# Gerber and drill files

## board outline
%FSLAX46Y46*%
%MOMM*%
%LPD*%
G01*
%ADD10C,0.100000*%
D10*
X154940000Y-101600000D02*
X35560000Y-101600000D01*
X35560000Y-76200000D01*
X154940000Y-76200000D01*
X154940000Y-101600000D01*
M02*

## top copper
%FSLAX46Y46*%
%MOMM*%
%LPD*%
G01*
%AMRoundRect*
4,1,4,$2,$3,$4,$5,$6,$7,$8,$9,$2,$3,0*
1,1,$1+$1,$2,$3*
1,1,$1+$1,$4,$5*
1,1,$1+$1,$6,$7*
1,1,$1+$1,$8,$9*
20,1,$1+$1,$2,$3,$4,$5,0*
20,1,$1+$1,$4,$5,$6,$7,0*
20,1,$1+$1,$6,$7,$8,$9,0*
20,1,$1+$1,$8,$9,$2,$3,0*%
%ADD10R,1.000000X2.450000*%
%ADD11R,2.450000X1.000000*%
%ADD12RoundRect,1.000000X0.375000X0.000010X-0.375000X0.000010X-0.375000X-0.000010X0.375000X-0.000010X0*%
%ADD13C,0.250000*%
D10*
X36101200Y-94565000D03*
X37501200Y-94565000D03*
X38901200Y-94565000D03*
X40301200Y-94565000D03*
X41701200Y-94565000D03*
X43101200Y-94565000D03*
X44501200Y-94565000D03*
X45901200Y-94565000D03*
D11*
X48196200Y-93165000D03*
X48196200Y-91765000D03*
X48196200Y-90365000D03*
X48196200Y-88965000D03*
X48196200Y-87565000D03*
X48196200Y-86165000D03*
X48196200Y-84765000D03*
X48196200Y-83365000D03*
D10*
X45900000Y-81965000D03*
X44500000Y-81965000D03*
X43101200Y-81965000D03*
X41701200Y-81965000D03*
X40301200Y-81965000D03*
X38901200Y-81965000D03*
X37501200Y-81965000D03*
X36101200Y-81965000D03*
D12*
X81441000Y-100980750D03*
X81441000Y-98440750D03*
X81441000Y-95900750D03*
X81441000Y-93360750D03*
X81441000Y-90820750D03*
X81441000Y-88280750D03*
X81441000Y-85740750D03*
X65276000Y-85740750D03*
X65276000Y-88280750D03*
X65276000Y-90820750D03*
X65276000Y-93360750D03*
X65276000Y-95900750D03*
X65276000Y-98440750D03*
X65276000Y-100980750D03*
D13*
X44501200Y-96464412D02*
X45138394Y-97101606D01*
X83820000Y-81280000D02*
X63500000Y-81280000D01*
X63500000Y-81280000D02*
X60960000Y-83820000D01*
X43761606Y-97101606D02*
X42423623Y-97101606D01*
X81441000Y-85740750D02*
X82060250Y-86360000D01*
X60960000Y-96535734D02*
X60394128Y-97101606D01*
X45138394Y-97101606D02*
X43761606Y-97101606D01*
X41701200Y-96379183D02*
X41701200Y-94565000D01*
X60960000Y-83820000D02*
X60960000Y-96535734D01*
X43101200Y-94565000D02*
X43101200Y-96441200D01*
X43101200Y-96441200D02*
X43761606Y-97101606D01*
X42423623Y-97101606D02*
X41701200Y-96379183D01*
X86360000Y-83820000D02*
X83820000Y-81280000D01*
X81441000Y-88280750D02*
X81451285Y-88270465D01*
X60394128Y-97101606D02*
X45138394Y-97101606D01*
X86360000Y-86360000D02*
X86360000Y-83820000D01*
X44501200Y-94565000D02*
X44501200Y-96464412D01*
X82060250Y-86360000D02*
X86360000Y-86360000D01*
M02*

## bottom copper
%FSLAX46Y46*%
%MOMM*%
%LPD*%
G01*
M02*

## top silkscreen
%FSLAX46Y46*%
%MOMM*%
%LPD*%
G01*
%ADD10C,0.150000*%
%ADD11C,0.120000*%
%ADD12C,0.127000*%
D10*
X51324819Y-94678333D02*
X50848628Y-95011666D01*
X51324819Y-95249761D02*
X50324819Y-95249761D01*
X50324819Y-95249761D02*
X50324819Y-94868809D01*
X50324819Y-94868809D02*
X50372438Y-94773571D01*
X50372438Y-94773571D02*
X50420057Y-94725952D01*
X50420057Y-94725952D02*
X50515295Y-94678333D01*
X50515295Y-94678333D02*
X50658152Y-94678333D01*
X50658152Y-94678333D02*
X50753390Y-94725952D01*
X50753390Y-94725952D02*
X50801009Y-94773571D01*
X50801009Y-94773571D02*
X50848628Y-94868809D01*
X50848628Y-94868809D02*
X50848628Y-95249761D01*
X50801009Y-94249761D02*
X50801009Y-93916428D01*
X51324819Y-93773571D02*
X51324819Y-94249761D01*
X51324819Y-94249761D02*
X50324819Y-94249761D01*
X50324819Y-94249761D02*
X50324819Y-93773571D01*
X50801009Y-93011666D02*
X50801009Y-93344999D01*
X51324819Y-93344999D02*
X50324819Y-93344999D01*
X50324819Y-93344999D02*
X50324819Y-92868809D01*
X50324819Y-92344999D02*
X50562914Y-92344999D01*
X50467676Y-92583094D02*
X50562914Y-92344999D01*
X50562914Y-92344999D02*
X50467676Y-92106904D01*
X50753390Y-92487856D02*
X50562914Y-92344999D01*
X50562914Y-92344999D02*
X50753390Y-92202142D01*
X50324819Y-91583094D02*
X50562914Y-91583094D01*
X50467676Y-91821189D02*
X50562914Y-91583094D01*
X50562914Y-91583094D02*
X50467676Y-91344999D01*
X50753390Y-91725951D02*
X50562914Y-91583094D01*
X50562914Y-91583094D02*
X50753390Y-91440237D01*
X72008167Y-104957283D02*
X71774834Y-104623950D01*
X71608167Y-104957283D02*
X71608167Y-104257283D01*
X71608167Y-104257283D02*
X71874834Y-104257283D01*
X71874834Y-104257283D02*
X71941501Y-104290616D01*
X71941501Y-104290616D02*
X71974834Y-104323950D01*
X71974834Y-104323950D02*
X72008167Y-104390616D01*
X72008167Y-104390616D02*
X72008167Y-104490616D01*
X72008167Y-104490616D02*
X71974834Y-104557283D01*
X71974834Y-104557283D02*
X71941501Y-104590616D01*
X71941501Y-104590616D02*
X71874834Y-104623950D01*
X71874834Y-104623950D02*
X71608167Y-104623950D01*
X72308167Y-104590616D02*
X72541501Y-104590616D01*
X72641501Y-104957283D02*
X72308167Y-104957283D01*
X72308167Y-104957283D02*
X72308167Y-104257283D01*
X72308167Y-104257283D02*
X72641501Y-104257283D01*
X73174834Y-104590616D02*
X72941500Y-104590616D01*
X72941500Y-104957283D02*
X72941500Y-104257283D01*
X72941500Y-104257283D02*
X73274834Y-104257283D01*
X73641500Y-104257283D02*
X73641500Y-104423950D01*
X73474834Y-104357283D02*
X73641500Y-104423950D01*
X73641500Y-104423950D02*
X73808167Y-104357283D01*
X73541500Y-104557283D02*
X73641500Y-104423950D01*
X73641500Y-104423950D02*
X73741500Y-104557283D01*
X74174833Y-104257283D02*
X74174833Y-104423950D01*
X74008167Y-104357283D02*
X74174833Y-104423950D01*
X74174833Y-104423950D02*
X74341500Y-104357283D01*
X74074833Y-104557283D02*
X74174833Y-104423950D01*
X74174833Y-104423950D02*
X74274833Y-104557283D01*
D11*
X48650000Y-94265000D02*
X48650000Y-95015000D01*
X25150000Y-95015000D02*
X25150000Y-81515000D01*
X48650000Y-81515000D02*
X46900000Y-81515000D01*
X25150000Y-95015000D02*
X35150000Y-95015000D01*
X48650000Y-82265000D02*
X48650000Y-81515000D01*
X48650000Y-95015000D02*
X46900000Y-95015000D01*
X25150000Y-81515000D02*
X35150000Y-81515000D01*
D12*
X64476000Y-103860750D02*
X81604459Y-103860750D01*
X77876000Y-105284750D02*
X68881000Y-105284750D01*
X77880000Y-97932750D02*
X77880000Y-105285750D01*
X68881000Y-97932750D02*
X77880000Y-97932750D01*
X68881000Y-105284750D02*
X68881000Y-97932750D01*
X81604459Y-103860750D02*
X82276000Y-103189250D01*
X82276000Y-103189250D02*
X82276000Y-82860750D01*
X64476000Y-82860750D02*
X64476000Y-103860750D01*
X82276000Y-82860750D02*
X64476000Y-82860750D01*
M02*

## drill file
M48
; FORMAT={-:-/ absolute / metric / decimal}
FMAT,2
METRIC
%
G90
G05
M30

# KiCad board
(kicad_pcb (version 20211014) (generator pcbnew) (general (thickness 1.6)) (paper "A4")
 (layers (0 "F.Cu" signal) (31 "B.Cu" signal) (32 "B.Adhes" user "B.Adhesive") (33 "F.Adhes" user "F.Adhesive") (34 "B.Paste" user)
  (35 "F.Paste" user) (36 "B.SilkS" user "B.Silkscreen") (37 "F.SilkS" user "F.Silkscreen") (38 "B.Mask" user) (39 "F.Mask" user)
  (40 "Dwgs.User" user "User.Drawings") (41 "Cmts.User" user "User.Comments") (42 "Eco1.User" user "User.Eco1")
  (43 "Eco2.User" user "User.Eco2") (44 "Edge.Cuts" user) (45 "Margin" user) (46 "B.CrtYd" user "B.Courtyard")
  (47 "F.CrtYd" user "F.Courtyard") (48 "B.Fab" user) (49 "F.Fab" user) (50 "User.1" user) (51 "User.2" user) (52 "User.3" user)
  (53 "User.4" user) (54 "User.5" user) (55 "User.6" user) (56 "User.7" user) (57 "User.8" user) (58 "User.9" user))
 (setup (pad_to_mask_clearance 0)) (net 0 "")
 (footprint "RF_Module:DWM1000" (layer "F.Cu") (at 36.9 88.265 90)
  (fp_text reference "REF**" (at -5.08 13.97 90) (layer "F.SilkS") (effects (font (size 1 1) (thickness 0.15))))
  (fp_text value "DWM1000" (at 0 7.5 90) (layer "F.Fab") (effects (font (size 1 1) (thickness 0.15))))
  (fp_line (start -6 11.75) (end -6.75 11.75) (layer "F.SilkS") (width 0.12))
  (fp_line (start -6.75 -11.75) (end 6.75 -11.75) (layer "F.SilkS") (width 0.12))
  (fp_line (start 6.75 11.75) (end 6.75 10) (layer "F.SilkS") (width 0.12))
  (fp_line (start -6.75 -11.75) (end -6.75 -1.75) (layer "F.SilkS") (width 0.12))
  (fp_line (start 6 11.75) (end 6.75 11.75) (layer "F.SilkS") (width 0.12))
  (fp_line (start -6.75 11.75) (end -6.75 10) (layer "F.SilkS") (width 0.12))
  (fp_line (start 6.75 -11.75) (end 6.75 -1.75) (layer "F.SilkS") (width 0.12))
  (pad "1" smd rect (at -6.3 -0.7988 180) (size 1 2.45) (layers "F.Cu" "F.Paste" "F.Mask"))
  (pad "2" smd rect (at -6.3 0.6012 180) (size 1 2.45) (layers "F.Cu" "F.Paste" "F.Mask"))
  (pad "3" smd rect (at -6.3 2.0012 180) (size 1 2.45) (layers "F.Cu" "F.Paste" "F.Mask"))
  (pad "4" smd rect (at -6.3 3.4012 180) (size 1 2.45) (layers "F.Cu" "F.Paste" "F.Mask"))
  (pad "5" smd rect (at -6.3 4.8012 180) (size 1 2.45) (layers "F.Cu" "F.Paste" "F.Mask"))
  (pad "6" smd rect (at -6.3 6.2012 180) (size 1 2.45) (layers "F.Cu" "F.Paste" "F.Mask"))
  (pad "7" smd rect (at -6.3 7.6012 180) (size 1 2.45) (layers "F.Cu" "F.Paste" "F.Mask"))
  (pad "8" smd rect (at -6.3 9.0012 180) (size 1 2.45) (layers "F.Cu" "F.Paste" "F.Mask"))
  (pad "9" smd rect (at -4.9 11.2962 90) (size 1 2.45) (layers "F.Cu" "F.Paste" "F.Mask"))
  (pad "10" smd rect (at -3.5 11.2962 90) (size 1 2.45) (layers "F.Cu" "F.Paste" "F.Mask"))
  (pad "11" smd rect (at -2.1 11.2962 90) (size 1 2.45) (layers "F.Cu" "F.Paste" "F.Mask"))
  (pad "12" smd rect (at -0.7 11.2962 90) (size 1 2.45) (layers "F.Cu" "F.Paste" "F.Mask"))
  (pad "13" smd rect (at 0.7 11.2962 90) (size 1 2.45) (layers "F.Cu" "F.Paste" "F.Mask"))
  (pad "14" smd rect (at 2.1 11.2962 90) (size 1 2.45) (layers "F.Cu" "F.Paste" "F.Mask"))
  (pad "15" smd rect (at 3.5 11.2962 90) (size 1 2.45) (layers "F.Cu" "F.Paste" "F.Mask"))
  (pad "16" smd rect (at 4.9 11.2962 90) (size 1 2.45) (layers "F.Cu" "F.Paste" "F.Mask"))
  (pad "17" smd rect (at 6.3 9 180) (size 1 2.45) (layers "F.Cu" "F.Paste" "F.Mask"))
  (pad "18" smd rect (at 6.3 7.6 180) (size 1 2.45) (layers "F.Cu" "F.Paste" "F.Mask"))
  (pad "19" smd rect (at 6.3 6.2012 180) (size 1 2.45) (layers "F.Cu" "F.Paste" "F.Mask"))
  (pad "20" smd rect (at 6.3 4.8012 180) (size 1 2.45) (layers "F.Cu" "F.Paste" "F.Mask"))
  (pad "21" smd rect (at 6.3 3.4012 180) (size 1 2.45) (layers "F.Cu" "F.Paste" "F.Mask"))
  (pad "22" smd rect (at 6.3 2.0012 180) (size 1 2.45) (layers "F.Cu" "F.Paste" "F.Mask"))
  (pad "23" smd rect (at 6.3 0.6012 180) (size 1 2.45) (layers "F.Cu" "F.Paste" "F.Mask"))
  (pad "24" smd rect (at 6.3 -0.7988 180) (size 1 2.45) (layers "F.Cu" "F.Paste" "F.Mask"))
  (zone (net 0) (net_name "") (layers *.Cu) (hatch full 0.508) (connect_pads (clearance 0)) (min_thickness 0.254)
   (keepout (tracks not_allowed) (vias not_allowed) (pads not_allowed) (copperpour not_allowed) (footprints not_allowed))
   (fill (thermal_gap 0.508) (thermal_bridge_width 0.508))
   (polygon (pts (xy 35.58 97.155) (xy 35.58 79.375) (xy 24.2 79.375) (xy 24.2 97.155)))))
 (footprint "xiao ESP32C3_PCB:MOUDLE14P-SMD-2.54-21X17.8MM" (layer "F.Cu") (at 82.276 82.86075 180)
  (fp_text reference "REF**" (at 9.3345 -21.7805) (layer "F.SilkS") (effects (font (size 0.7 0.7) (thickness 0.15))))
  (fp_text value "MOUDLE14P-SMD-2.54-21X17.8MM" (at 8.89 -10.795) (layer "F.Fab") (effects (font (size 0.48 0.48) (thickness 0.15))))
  (fp_line (start 17.8 -21) (end 0.671541 -21) (layer "F.SilkS") (width 0.127))
  (fp_line (start 4.4 -22.424) (end 13.395 -22.424) (layer "F.SilkS") (width 0.127))
  (fp_line (start 4.396 -15.072) (end 4.396 -22.425) (layer "F.SilkS") (width 0.127))
  (fp_line (start 13.395 -15.072) (end 4.396 -15.072) (layer "F.SilkS") (width 0.127))
  (fp_line (start 13.395 -22.424) (end 13.395 -15.072) (layer "F.SilkS") (width 0.127))
  (fp_line (start 0.671541 -21) (end 0 -20.3285) (layer "F.SilkS") (width 0.127))
  (fp_line (start 0 -20.3285) (end 0 0) (layer "F.SilkS") (width 0.127))
  (fp_line (start 17.8 0) (end 17.8 -21) (layer "F.SilkS") (width 0.127))
  (fp_line (start 0 0) (end 17.8 0) (layer "F.SilkS") (width 0.127))
  (pad "1" smd roundrect locked (at 0.835 -18.12 180) (size 2.75 2) (layers "F.Cu" "F.Paste" "F.Mask") (roundrect_rratio 0.5))
  (pad "2" smd roundrect locked (at 0.835 -15.58 180) (size 2.75 2) (layers "F.Cu" "F.Paste" "F.Mask") (roundrect_rratio 0.5))
  (pad "3" smd roundrect locked (at 0.835 -13.04 180) (size 2.75 2) (layers "F.Cu" "F.Paste" "F.Mask") (roundrect_rratio 0.5))
  (pad "4" smd roundrect locked (at 0.835 -10.5 180) (size 2.75 2) (layers "F.Cu" "F.Paste" "F.Mask") (roundrect_rratio 0.5))
  (pad "5" smd roundrect locked (at 0.835 -7.96 180) (size 2.75 2) (layers "F.Cu" "F.Paste" "F.Mask") (roundrect_rratio 0.5))
  (pad "6" smd roundrect locked (at 0.835 -5.42 180) (size 2.75 2) (layers "F.Cu" "F.Paste" "F.Mask") (roundrect_rratio 0.5))
  (pad "7" smd roundrect locked (at 0.835 -2.88 180) (size 2.75 2) (layers "F.Cu" "F.Paste" "F.Mask") (roundrect_rratio 0.5))
  (pad "8" smd roundrect locked (at 17 -2.88 180) (size 2.75 2) (layers "F.Cu" "F.Paste" "F.Mask") (roundrect_rratio 0.5))
  (pad "9" smd roundrect locked (at 17 -5.42 180) (size 2.75 2) (layers "F.Cu" "F.Paste" "F.Mask") (roundrect_rratio 0.5))
  (pad "10" smd roundrect locked (at 17 -7.96 180) (size 2.75 2) (layers "F.Cu" "F.Paste" "F.Mask") (roundrect_rratio 0.5))
  (pad "11" smd roundrect locked (at 17 -10.5 180) (size 2.75 2) (layers "F.Cu" "F.Paste" "F.Mask") (roundrect_rratio 0.5))
  (pad "12" smd roundrect locked (at 17 -13.04 180) (size 2.75 2) (layers "F.Cu" "F.Paste" "F.Mask") (roundrect_rratio 0.5))
  (pad "13" smd roundrect locked (at 17 -15.58 180) (size 2.75 2) (layers "F.Cu" "F.Paste" "F.Mask") (roundrect_rratio 0.5))
  (pad "14" smd roundrect locked (at 17 -18.12 180) (size 2.75 2) (layers "F.Cu" "F.Paste" "F.Mask") (roundrect_rratio 0.5))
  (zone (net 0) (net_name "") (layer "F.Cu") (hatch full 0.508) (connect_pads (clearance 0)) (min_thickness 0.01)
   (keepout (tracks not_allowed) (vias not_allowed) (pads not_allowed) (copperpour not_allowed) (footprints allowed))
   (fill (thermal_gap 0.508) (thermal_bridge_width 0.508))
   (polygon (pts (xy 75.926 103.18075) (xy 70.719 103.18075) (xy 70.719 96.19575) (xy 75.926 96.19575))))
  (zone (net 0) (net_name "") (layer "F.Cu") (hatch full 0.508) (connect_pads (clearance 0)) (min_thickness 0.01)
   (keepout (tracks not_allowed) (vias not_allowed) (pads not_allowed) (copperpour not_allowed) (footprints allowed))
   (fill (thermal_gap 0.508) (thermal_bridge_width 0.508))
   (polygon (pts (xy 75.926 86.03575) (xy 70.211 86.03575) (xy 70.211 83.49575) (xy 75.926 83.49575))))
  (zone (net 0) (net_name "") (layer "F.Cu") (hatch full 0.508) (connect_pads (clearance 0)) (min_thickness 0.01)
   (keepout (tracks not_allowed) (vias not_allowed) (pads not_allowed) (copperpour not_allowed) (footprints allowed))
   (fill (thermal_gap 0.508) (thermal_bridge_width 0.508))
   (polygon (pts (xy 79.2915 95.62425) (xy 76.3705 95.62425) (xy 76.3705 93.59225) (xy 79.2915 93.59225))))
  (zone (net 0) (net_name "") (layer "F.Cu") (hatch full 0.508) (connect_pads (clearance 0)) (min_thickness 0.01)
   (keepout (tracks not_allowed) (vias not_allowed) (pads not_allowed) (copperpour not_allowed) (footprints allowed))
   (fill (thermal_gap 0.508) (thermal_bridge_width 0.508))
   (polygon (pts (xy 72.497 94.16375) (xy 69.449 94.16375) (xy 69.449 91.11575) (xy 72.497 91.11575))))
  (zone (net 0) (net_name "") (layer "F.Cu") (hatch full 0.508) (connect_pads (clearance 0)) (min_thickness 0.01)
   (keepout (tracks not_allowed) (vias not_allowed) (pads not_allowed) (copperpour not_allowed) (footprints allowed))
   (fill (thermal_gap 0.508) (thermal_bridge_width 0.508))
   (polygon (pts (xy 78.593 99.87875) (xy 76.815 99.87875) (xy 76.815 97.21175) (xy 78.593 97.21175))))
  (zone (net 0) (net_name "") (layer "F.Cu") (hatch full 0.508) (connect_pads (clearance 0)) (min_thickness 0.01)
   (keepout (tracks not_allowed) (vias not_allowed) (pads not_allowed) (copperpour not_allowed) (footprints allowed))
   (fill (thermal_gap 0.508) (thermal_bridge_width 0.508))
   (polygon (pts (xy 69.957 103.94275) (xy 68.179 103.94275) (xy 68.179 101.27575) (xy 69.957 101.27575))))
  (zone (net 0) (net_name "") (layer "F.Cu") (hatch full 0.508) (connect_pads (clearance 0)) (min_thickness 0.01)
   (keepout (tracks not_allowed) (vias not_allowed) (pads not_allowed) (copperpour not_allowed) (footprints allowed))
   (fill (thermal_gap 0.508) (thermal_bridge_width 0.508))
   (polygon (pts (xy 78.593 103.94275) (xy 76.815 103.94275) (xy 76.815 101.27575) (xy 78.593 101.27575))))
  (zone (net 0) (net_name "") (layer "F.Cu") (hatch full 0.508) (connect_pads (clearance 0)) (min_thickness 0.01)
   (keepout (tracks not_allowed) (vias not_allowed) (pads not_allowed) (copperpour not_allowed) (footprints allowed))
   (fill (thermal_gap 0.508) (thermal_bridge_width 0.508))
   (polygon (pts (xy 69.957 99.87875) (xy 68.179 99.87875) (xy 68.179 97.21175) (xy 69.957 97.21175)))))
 (gr_poly (pts (xy 154.94 101.6) (xy 35.56 101.6) (xy 35.56 76.2) (xy 154.94 76.2)) (layer "Edge.Cuts") (width 0.1) (fill none))
 (segment (start 44.5012 96.464412) (end 45.138394 97.101606) (width 0.25) (layer "F.Cu") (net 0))
 (segment (start 83.82 81.28) (end 63.5 81.28) (width 0.25) (layer "F.Cu") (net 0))
 (segment (start 63.5 81.28) (end 60.96 83.82) (width 0.25) (layer "F.Cu") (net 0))
 (segment (start 43.761606 97.101606) (end 42.423623 97.101606) (width 0.25) (layer "F.Cu") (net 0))
 (segment (start 81.441 85.74075) (end 82.06025 86.36) (width 0.25) (layer "F.Cu") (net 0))
 (segment (start 60.96 96.535734) (end 60.394128 97.101606) (width 0.25) (layer "F.Cu") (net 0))
 (segment (start 45.138394 97.101606) (end 43.761606 97.101606) (width 0.25) (layer "F.Cu") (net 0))
 (segment (start 41.7012 96.379183) (end 41.7012 94.565) (width 0.25) (layer "F.Cu") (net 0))
 (segment (start 60.96 83.82) (end 60.96 96.535734) (width 0.25) (layer "F.Cu") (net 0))
 (segment (start 43.1012 94.565) (end 43.1012 96.4412) (width 0.25) (layer "F.Cu") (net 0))
 (segment (start 43.1012 96.4412) (end 43.761606 97.101606) (width 0.25) (layer "F.Cu") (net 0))
 (segment (start 42.423623 97.101606) (end 41.7012 96.379183) (width 0.25) (layer "F.Cu") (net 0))
 (segment (start 86.36 83.82) (end 83.82 81.28) (width 0.25) (layer "F.Cu") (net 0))
 (segment (start 81.441 88.28075) (end 81.451285 88.270465) (width 0.25) (layer "F.Cu") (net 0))
 (segment (start 60.394128 97.101606) (end 45.138394 97.101606) (width 0.25) (layer "F.Cu") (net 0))
 (segment (start 86.36 86.36) (end 86.36 83.82) (width 0.25) (layer "F.Cu") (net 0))
 (segment (start 44.5012 94.565) (end 44.5012 96.464412) (width 0.25) (layer "F.Cu") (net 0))
 (segment (start 82.06025 86.36) (end 86.36 86.36) (width 0.25) (layer "F.Cu") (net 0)))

